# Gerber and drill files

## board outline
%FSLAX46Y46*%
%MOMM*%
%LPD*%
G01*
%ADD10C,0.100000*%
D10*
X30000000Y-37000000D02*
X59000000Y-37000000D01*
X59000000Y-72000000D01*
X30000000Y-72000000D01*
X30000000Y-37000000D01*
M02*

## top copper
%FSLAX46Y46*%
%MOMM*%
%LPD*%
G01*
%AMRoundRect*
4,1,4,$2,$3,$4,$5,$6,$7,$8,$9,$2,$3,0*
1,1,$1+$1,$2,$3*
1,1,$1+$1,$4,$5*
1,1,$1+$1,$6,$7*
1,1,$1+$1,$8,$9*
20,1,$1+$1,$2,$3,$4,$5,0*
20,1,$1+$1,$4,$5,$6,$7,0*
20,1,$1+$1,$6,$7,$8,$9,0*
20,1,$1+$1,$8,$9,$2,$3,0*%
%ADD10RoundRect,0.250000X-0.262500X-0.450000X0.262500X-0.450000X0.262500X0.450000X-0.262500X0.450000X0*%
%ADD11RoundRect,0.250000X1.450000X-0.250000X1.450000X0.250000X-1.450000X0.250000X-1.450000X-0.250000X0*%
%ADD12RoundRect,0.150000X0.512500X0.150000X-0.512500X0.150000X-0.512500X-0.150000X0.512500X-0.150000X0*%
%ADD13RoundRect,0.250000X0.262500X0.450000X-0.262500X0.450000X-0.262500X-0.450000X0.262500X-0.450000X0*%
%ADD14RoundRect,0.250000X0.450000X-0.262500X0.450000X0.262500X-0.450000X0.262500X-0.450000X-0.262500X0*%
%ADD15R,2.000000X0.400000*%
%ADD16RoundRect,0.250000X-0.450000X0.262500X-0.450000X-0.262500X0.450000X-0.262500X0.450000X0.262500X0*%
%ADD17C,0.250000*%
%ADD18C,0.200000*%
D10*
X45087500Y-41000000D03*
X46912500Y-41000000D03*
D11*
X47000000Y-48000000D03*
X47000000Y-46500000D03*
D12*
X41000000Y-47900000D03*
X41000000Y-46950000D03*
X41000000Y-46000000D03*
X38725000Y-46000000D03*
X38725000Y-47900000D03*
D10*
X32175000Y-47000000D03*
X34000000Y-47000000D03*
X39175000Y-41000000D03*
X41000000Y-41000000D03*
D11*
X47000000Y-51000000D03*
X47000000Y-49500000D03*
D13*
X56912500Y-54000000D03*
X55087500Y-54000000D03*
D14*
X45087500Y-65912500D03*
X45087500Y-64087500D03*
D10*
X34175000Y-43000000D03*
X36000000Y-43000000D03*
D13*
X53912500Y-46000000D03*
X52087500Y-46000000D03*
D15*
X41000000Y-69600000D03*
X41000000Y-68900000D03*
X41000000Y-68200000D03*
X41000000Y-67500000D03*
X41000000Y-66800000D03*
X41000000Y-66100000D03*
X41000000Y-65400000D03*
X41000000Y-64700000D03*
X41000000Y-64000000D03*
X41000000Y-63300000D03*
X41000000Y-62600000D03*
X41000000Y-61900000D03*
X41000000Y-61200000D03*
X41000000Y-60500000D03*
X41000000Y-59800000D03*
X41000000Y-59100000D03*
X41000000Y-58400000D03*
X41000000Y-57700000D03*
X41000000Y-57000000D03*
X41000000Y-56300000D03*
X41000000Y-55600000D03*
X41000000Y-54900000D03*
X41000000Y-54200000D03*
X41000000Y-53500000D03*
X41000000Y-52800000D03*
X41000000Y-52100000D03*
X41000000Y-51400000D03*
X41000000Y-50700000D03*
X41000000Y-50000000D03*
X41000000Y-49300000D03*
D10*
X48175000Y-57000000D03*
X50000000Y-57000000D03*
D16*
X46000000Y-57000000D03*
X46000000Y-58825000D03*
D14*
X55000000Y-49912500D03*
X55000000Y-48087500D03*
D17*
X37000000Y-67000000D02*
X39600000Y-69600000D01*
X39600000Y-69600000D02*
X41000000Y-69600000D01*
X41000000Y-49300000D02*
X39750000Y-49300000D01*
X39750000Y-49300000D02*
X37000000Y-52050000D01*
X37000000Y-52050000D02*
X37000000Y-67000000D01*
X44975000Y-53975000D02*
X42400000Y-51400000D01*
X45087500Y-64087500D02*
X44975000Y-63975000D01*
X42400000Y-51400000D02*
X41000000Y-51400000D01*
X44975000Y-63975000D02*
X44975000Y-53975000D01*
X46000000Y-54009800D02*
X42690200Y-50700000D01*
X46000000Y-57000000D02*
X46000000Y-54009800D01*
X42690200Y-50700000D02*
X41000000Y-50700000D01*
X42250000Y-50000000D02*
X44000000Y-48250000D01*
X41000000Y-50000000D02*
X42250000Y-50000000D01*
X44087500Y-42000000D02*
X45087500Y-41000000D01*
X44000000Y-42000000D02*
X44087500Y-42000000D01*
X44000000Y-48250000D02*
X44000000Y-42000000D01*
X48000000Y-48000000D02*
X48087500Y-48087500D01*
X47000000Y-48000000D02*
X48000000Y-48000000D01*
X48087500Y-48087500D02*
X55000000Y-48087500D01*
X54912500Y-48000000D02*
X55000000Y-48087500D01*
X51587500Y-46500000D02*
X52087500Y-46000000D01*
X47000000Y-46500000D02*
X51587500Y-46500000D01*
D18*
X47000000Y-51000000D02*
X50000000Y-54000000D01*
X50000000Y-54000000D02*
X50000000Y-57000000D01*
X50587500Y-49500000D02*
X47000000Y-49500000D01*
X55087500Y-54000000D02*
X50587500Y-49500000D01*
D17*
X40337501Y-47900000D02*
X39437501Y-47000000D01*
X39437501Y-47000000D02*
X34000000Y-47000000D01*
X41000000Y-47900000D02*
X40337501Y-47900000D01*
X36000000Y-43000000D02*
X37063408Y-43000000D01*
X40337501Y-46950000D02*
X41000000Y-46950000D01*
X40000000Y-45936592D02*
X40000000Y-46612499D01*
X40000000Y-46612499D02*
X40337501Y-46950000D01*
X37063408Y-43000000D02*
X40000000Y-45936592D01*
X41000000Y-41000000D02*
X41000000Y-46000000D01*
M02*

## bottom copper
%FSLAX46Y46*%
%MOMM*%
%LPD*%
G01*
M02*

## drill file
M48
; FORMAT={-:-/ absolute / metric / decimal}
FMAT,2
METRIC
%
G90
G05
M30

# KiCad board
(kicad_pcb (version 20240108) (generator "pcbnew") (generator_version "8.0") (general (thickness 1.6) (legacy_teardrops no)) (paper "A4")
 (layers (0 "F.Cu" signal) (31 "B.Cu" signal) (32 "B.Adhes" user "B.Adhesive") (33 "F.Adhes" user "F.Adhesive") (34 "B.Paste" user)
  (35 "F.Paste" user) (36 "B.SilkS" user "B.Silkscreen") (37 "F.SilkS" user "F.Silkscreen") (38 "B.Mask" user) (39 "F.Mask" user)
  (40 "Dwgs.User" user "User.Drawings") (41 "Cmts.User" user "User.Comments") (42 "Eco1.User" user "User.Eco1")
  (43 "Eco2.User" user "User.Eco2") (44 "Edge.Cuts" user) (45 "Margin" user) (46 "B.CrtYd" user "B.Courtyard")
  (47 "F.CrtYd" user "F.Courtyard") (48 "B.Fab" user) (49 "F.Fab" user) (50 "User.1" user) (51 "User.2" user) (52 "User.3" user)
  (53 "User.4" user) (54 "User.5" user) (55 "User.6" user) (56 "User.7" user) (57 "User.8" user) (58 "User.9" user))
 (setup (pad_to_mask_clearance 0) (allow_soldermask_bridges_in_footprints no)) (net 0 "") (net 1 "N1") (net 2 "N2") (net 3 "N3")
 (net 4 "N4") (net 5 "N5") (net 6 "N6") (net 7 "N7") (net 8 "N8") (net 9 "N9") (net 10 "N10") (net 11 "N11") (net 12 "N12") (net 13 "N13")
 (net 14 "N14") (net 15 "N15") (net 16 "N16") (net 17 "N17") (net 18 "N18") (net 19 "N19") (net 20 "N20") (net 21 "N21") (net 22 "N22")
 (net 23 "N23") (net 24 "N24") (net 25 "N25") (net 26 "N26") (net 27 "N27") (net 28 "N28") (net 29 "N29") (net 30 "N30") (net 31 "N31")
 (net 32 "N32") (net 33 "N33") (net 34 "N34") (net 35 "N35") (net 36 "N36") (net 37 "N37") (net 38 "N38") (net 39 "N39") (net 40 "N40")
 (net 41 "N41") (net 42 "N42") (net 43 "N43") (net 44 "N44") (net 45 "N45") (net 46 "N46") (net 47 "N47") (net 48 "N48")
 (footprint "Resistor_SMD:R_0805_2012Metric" (layer "F.Cu") (at 46 41)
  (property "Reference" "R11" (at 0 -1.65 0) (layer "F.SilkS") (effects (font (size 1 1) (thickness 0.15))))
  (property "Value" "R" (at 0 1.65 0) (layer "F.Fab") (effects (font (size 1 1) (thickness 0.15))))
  (pad "1" smd roundrect (at -0.9125 0) (size 1.025 1.4) (layers "F.Cu" "F.Paste" "F.Mask") (roundrect_rratio 0.243902) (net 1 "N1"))
  (pad "2" smd roundrect (at 0.9125 0) (size 1.025 1.4) (layers "F.Cu" "F.Paste" "F.Mask") (roundrect_rratio 0.243902) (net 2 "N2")))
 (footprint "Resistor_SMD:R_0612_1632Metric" (layer "F.Cu") (at 47 47.25 90)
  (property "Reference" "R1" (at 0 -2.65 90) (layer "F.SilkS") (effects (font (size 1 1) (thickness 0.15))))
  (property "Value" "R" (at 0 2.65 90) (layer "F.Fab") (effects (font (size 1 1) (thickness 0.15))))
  (pad "1" smd roundrect (at -0.75 0 90) (size 1 3.4) (layers "F.Cu" "F.Paste" "F.Mask") (roundrect_rratio 0.25) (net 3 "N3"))
  (pad "2" smd roundrect (at 0.75 0 90) (size 1 3.4) (layers "F.Cu" "F.Paste" "F.Mask") (roundrect_rratio 0.25) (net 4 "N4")))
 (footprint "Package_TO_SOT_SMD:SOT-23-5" (layer "F.Cu") (at 39.8625 46.95 180)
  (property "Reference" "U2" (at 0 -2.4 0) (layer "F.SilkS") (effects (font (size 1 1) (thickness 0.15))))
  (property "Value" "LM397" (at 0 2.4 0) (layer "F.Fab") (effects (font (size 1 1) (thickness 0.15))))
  (pad "1" smd roundrect (at -1.1375 -0.95 180) (size 1.325 0.6) (layers "F.Cu" "F.Paste" "F.Mask") (roundrect_rratio 0.25) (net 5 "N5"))
  (pad "2" smd roundrect (at -1.1375 0 180) (size 1.325 0.6) (layers "F.Cu" "F.Paste" "F.Mask") (roundrect_rratio 0.25) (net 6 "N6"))
  (pad "3" smd roundrect (at -1.1375 0.95 180) (size 1.325 0.6) (layers "F.Cu" "F.Paste" "F.Mask") (roundrect_rratio 0.25) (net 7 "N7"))
  (pad "4" smd roundrect (at 1.1375 0.95 180) (size 1.325 0.6) (layers "F.Cu" "F.Paste" "F.Mask") (roundrect_rratio 0.25) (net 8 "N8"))
  (pad "5" smd roundrect (at 1.1375 -0.95 180) (size 1.325 0.6) (layers "F.Cu" "F.Paste" "F.Mask") (roundrect_rratio 0.25) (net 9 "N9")))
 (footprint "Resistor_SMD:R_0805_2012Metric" (layer "F.Cu") (at 33.0875 47)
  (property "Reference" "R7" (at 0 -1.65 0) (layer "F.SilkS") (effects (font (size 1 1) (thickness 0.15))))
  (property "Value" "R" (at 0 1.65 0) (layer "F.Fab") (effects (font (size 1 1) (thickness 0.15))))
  (pad "1" smd roundrect (at -0.9125 0) (size 1.025 1.4) (layers "F.Cu" "F.Paste" "F.Mask") (roundrect_rratio 0.243902) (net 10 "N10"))
  (pad "2" smd roundrect (at 0.9125 0) (size 1.025 1.4) (layers "F.Cu" "F.Paste" "F.Mask") (roundrect_rratio 0.243902) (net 5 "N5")))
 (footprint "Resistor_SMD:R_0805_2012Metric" (layer "F.Cu") (at 40.0875 41)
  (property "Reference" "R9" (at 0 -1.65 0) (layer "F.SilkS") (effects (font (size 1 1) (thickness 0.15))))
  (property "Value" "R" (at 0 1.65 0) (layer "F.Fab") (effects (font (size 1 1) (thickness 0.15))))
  (pad "1" smd roundrect (at -0.9125 0) (size 1.025 1.4) (layers "F.Cu" "F.Paste" "F.Mask") (roundrect_rratio 0.243902) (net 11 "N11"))
  (pad "2" smd roundrect (at 0.9125 0) (size 1.025 1.4) (layers "F.Cu" "F.Paste" "F.Mask") (roundrect_rratio 0.243902) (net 7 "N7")))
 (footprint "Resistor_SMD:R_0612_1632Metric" (layer "F.Cu") (at 47 50.25 90)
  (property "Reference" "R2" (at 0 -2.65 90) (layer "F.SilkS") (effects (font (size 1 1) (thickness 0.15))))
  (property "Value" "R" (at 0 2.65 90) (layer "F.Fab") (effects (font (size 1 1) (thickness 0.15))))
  (pad "1" smd roundrect (at -0.75 0 90) (size 1 3.4) (layers "F.Cu" "F.Paste" "F.Mask") (roundrect_rratio 0.25) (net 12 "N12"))
  (pad "2" smd roundrect (at 0.75 0 90) (size 1 3.4) (layers "F.Cu" "F.Paste" "F.Mask") (roundrect_rratio 0.25) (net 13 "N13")))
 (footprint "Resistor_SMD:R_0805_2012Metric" (layer "F.Cu") (at 56 54 180)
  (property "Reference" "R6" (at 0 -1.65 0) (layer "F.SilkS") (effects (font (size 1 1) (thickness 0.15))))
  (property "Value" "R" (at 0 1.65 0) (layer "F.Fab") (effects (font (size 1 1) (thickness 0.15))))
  (pad "1" smd roundrect (at -0.9125 0 180) (size 1.025 1.4) (layers "F.Cu" "F.Paste" "F.Mask") (roundrect_rratio 0.243902) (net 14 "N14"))
  (pad "2" smd roundrect (at 0.9125 0 180) (size 1.025 1.4) (layers "F.Cu" "F.Paste" "F.Mask") (roundrect_rratio 0.243902) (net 13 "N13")))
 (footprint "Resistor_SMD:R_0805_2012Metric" (layer "F.Cu") (at 45.0875 65 90)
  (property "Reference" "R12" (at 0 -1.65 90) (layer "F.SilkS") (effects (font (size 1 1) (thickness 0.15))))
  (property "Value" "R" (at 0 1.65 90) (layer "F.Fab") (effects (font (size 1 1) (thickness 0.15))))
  (pad "1" smd roundrect (at -0.9125 0 90) (size 1.025 1.4) (layers "F.Cu" "F.Paste" "F.Mask") (roundrect_rratio 0.243902) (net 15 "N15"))
  (pad "2" smd roundrect (at 0.9125 0 90) (size 1.025 1.4) (layers "F.Cu" "F.Paste" "F.Mask") (roundrect_rratio 0.243902) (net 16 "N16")))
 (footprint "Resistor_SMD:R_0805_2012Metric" (layer "F.Cu") (at 35.0875 43)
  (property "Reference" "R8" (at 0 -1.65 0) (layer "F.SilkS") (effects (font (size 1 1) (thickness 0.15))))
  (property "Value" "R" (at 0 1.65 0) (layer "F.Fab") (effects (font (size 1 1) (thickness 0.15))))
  (pad "1" smd roundrect (at -0.9125 0) (size 1.025 1.4) (layers "F.Cu" "F.Paste" "F.Mask") (roundrect_rratio 0.243902) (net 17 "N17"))
  (pad "2" smd roundrect (at 0.9125 0) (size 1.025 1.4) (layers "F.Cu" "F.Paste" "F.Mask") (roundrect_rratio 0.243902) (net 6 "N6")))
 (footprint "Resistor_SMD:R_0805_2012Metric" (layer "F.Cu") (at 53 46 180)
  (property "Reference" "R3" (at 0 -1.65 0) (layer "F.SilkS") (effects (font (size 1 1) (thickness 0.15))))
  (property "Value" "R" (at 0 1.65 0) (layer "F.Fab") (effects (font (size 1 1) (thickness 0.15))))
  (pad "1" smd roundrect (at -0.9125 0 180) (size 1.025 1.4) (layers "F.Cu" "F.Paste" "F.Mask") (roundrect_rratio 0.243902) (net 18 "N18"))
  (pad "2" smd roundrect (at 0.9125 0 180) (size 1.025 1.4) (layers "F.Cu" "F.Paste" "F.Mask") (roundrect_rratio 0.243902) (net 4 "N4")))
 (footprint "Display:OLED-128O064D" (layer "F.Cu") (at 41 59.45 90)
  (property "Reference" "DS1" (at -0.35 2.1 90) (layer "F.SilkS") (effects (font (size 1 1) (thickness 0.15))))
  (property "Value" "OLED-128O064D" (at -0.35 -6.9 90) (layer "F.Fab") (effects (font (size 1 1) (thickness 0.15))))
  (pad "1" smd rect (at -10.15 0 90) (size 0.4 2) (layers "F.Cu" "F.Paste" "F.Mask") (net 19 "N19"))
  (pad "2" smd rect (at -9.45 0 90) (size 0.4 2) (layers "F.Cu" "F.Paste" "F.Mask") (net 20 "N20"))
  (pad "3" smd rect (at -8.75 0 90) (size 0.4 2) (layers "F.Cu" "F.Paste" "F.Mask") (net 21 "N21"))
  (pad "4" smd rect (at -8.05 0 90) (size 0.4 2) (layers "F.Cu" "F.Paste" "F.Mask") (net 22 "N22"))
  (pad "5" smd rect (at -7.35 0 90) (size 0.4 2) (layers "F.Cu" "F.Paste" "F.Mask") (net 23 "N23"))
  (pad "6" smd rect (at -6.65 0 90) (size 0.4 2) (layers "F.Cu" "F.Paste" "F.Mask") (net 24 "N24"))
  (pad "7" smd rect (at -5.95 0 90) (size 0.4 2) (layers "F.Cu" "F.Paste" "F.Mask") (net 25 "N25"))
  (pad "8" smd rect (at -5.25 0 90) (size 0.4 2) (layers "F.Cu" "F.Paste" "F.Mask") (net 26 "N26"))
  (pad "9" smd rect (at -4.55 0 90) (size 0.4 2) (layers "F.Cu" "F.Paste" "F.Mask") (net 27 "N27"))
  (pad "10" smd rect (at -3.85 0 90) (size 0.4 2) (layers "F.Cu" "F.Paste" "F.Mask") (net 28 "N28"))
  (pad "11" smd rect (at -3.15 0 90) (size 0.4 2) (layers "F.Cu" "F.Paste" "F.Mask") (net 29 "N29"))
  (pad "12" smd rect (at -2.45 0 90) (size 0.4 2) (layers "F.Cu" "F.Paste" "F.Mask") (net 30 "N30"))
  (pad "13" smd rect (at -1.75 0 90) (size 0.4 2) (layers "F.Cu" "F.Paste" "F.Mask") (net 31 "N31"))
  (pad "14" smd rect (at -1.05 0 90) (size 0.4 2) (layers "F.Cu" "F.Paste" "F.Mask") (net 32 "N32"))
  (pad "15" smd rect (at -0.35 0 90) (size 0.4 2) (layers "F.Cu" "F.Paste" "F.Mask") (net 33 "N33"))
  (pad "16" smd rect (at 0.35 0 90) (size 0.4 2) (layers "F.Cu" "F.Paste" "F.Mask") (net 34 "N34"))
  (pad "17" smd rect (at 1.05 0 90) (size 0.4 2) (layers "F.Cu" "F.Paste" "F.Mask") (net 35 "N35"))
  (pad "18" smd rect (at 1.75 0 90) (size 0.4 2) (layers "F.Cu" "F.Paste" "F.Mask") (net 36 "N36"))
  (pad "19" smd rect (at 2.45 0 90) (size 0.4 2) (layers "F.Cu" "F.Paste" "F.Mask") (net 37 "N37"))
  (pad "20" smd rect (at 3.15 0 90) (size 0.4 2) (layers "F.Cu" "F.Paste" "F.Mask") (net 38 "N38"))
  (pad "21" smd rect (at 3.85 0 90) (size 0.4 2) (layers "F.Cu" "F.Paste" "F.Mask") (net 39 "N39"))
  (pad "22" smd rect (at 4.55 0 90) (size 0.4 2) (layers "F.Cu" "F.Paste" "F.Mask") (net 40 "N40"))
  (pad "23" smd rect (at 5.25 0 90) (size 0.4 2) (layers "F.Cu" "F.Paste" "F.Mask") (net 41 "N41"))
  (pad "24" smd rect (at 5.95 0 90) (size 0.4 2) (layers "F.Cu" "F.Paste" "F.Mask") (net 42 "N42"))
  (pad "25" smd rect (at 6.65 0 90) (size 0.4 2) (layers "F.Cu" "F.Paste" "F.Mask") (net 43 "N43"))
  (pad "26" smd rect (at 7.35 0 90) (size 0.4 2) (layers "F.Cu" "F.Paste" "F.Mask") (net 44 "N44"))
  (pad "27" smd rect (at 8.05 0 90) (size 0.4 2) (layers "F.Cu" "F.Paste" "F.Mask") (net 16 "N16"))
  (pad "28" smd rect (at 8.75 0 90) (size 0.4 2) (layers "F.Cu" "F.Paste" "F.Mask") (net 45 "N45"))
  (pad "29" smd rect (at 9.45 0 90) (size 0.4 2) (layers "F.Cu" "F.Paste" "F.Mask") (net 1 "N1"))
  (pad "30" smd rect (at 10.15 0 90) (size 0.4 2) (layers "F.Cu" "F.Paste" "F.Mask") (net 19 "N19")))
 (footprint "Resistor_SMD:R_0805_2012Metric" (layer "F.Cu") (at 49.0875 57)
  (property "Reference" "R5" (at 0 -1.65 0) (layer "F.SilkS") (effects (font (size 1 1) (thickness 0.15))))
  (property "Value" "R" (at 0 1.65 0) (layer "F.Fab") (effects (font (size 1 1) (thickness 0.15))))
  (pad "1" smd roundrect (at -0.9125 0) (size 1.025 1.4) (layers "F.Cu" "F.Paste" "F.Mask") (roundrect_rratio 0.243902) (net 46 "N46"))
  (pad "2" smd roundrect (at 0.9125 0) (size 1.025 1.4) (layers "F.Cu" "F.Paste" "F.Mask") (roundrect_rratio 0.243902) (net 12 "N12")))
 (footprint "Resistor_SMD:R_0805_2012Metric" (layer "F.Cu") (at 46 57.9125 -90)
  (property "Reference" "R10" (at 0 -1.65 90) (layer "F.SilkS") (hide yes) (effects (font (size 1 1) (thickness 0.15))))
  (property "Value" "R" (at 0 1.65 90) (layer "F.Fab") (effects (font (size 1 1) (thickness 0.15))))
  (pad "1" smd roundrect (at -0.9125 0 270) (size 1.025 1.4) (layers "F.Cu" "F.Paste" "F.Mask") (roundrect_rratio 0.243902) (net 45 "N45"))
  (pad "2" smd roundrect (at 0.9125 0 270) (size 1.025 1.4) (layers "F.Cu" "F.Paste" "F.Mask") (roundrect_rratio 0.243902) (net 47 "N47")))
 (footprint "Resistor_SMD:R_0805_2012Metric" (layer "F.Cu") (at 55 49 90)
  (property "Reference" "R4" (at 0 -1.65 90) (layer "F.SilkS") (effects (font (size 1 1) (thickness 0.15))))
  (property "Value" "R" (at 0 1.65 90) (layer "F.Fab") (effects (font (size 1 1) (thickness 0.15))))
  (pad "1" smd roundrect (at -0.9125 0 90) (size 1.025 1.4) (layers "F.Cu" "F.Paste" "F.Mask") (roundrect_rratio 0.243902) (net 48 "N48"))
  (pad "2" smd roundrect (at 0.9125 0 90) (size 1.025 1.4) (layers "F.Cu" "F.Paste" "F.Mask") (roundrect_rratio 0.243902) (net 3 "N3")))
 (gr_rect (start 30 37) (end 59 72) (stroke (width 0.1) (type default)) (fill none) (layer "Edge.Cuts"))
 (segment (start 37 67) (end 39.6 69.6) (width 0.25) (layer "F.Cu") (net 19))
 (segment (start 39.6 69.6) (end 41 69.6) (width 0.25) (layer "F.Cu") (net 19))
 (segment (start 41 49.3) (end 39.75 49.3) (width 0.25) (layer "F.Cu") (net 19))
 (segment (start 39.75 49.3) (end 37 52.05) (width 0.25) (layer "F.Cu") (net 19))
 (segment (start 37 52.05) (end 37 67) (width 0.25) (layer "F.Cu") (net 19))
 (segment (start 44.975 53.975) (end 42.4 51.4) (width 0.25) (layer "F.Cu") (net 16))
 (segment (start 45.0875 64.0875) (end 44.975 63.975) (width 0.25) (layer "F.Cu") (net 16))
 (segment (start 42.4 51.4) (end 41 51.4) (width 0.25) (layer "F.Cu") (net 16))
 (segment (start 44.975 63.975) (end 44.975 53.975) (width 0.25) (layer "F.Cu") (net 16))
 (segment (start 46 54.0098) (end 42.6902 50.7) (width 0.25) (layer "F.Cu") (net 45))
 (segment (start 46 57) (end 46 54.0098) (width 0.25) (layer "F.Cu") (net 45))
 (segment (start 42.6902 50.7) (end 41 50.7) (width 0.25) (layer "F.Cu") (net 45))
 (segment (start 42.25 50) (end 44 48.25) (width 0.25) (layer "F.Cu") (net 1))
 (segment (start 41 50) (end 42.25 50) (width 0.25) (layer "F.Cu") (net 1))
 (segment (start 44.0875 42) (end 45.0875 41) (width 0.25) (layer "F.Cu") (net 1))
 (segment (start 44 42) (end 44.0875 42) (width 0.25) (layer "F.Cu") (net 1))
 (segment (start 44 48.25) (end 44 42) (width 0.25) (layer "F.Cu") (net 1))
 (segment (start 48 48) (end 48.0875 48.0875) (width 0.25) (layer "F.Cu") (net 3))
 (segment (start 47 48) (end 48 48) (width 0.25) (layer "F.Cu") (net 3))
 (segment (start 48.0875 48.0875) (end 55 48.0875) (width 0.25) (layer "F.Cu") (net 3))
 (segment (start 54.9125 48) (end 55 48.0875) (width 0.25) (layer "F.Cu") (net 3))
 (segment (start 51.5875 46.5) (end 52.0875 46) (width 0.25) (layer "F.Cu") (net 4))
 (segment (start 47 46.5) (end 51.5875 46.5) (width 0.25) (layer "F.Cu") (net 4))
 (segment (start 47 51) (end 50 54) (width 0.2) (layer "F.Cu") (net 12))
 (segment (start 50 54) (end 50 57) (width 0.2) (layer "F.Cu") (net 12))
 (segment (start 50.5875 49.5) (end 47 49.5) (width 0.2) (layer "F.Cu") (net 13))
 (segment (start 55.0875 54) (end 50.5875 49.5) (width 0.2) (layer "F.Cu") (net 13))
 (segment (start 40.337501 47.9) (end 39.437501 47) (width 0.25) (layer "F.Cu") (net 5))
 (segment (start 39.437501 47) (end 34 47) (width 0.25) (layer "F.Cu") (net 5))
 (segment (start 41 47.9) (end 40.337501 47.9) (width 0.25) (layer "F.Cu") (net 5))
 (segment (start 36 43) (end 37.063408 43) (width 0.25) (layer "F.Cu") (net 6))
 (segment (start 40.337501 46.95) (end 41 46.95) (width 0.25) (layer "F.Cu") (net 6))
 (segment (start 40 45.936592) (end 40 46.612499) (width 0.25) (layer "F.Cu") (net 6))
 (segment (start 40 46.612499) (end 40.337501 46.95) (width 0.25) (layer "F.Cu") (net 6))
 (segment (start 37.063408 43) (end 40 45.936592) (width 0.25) (layer "F.Cu") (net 6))
 (segment (start 41 41) (end 41 46) (width 0.25) (layer "F.Cu") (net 7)))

